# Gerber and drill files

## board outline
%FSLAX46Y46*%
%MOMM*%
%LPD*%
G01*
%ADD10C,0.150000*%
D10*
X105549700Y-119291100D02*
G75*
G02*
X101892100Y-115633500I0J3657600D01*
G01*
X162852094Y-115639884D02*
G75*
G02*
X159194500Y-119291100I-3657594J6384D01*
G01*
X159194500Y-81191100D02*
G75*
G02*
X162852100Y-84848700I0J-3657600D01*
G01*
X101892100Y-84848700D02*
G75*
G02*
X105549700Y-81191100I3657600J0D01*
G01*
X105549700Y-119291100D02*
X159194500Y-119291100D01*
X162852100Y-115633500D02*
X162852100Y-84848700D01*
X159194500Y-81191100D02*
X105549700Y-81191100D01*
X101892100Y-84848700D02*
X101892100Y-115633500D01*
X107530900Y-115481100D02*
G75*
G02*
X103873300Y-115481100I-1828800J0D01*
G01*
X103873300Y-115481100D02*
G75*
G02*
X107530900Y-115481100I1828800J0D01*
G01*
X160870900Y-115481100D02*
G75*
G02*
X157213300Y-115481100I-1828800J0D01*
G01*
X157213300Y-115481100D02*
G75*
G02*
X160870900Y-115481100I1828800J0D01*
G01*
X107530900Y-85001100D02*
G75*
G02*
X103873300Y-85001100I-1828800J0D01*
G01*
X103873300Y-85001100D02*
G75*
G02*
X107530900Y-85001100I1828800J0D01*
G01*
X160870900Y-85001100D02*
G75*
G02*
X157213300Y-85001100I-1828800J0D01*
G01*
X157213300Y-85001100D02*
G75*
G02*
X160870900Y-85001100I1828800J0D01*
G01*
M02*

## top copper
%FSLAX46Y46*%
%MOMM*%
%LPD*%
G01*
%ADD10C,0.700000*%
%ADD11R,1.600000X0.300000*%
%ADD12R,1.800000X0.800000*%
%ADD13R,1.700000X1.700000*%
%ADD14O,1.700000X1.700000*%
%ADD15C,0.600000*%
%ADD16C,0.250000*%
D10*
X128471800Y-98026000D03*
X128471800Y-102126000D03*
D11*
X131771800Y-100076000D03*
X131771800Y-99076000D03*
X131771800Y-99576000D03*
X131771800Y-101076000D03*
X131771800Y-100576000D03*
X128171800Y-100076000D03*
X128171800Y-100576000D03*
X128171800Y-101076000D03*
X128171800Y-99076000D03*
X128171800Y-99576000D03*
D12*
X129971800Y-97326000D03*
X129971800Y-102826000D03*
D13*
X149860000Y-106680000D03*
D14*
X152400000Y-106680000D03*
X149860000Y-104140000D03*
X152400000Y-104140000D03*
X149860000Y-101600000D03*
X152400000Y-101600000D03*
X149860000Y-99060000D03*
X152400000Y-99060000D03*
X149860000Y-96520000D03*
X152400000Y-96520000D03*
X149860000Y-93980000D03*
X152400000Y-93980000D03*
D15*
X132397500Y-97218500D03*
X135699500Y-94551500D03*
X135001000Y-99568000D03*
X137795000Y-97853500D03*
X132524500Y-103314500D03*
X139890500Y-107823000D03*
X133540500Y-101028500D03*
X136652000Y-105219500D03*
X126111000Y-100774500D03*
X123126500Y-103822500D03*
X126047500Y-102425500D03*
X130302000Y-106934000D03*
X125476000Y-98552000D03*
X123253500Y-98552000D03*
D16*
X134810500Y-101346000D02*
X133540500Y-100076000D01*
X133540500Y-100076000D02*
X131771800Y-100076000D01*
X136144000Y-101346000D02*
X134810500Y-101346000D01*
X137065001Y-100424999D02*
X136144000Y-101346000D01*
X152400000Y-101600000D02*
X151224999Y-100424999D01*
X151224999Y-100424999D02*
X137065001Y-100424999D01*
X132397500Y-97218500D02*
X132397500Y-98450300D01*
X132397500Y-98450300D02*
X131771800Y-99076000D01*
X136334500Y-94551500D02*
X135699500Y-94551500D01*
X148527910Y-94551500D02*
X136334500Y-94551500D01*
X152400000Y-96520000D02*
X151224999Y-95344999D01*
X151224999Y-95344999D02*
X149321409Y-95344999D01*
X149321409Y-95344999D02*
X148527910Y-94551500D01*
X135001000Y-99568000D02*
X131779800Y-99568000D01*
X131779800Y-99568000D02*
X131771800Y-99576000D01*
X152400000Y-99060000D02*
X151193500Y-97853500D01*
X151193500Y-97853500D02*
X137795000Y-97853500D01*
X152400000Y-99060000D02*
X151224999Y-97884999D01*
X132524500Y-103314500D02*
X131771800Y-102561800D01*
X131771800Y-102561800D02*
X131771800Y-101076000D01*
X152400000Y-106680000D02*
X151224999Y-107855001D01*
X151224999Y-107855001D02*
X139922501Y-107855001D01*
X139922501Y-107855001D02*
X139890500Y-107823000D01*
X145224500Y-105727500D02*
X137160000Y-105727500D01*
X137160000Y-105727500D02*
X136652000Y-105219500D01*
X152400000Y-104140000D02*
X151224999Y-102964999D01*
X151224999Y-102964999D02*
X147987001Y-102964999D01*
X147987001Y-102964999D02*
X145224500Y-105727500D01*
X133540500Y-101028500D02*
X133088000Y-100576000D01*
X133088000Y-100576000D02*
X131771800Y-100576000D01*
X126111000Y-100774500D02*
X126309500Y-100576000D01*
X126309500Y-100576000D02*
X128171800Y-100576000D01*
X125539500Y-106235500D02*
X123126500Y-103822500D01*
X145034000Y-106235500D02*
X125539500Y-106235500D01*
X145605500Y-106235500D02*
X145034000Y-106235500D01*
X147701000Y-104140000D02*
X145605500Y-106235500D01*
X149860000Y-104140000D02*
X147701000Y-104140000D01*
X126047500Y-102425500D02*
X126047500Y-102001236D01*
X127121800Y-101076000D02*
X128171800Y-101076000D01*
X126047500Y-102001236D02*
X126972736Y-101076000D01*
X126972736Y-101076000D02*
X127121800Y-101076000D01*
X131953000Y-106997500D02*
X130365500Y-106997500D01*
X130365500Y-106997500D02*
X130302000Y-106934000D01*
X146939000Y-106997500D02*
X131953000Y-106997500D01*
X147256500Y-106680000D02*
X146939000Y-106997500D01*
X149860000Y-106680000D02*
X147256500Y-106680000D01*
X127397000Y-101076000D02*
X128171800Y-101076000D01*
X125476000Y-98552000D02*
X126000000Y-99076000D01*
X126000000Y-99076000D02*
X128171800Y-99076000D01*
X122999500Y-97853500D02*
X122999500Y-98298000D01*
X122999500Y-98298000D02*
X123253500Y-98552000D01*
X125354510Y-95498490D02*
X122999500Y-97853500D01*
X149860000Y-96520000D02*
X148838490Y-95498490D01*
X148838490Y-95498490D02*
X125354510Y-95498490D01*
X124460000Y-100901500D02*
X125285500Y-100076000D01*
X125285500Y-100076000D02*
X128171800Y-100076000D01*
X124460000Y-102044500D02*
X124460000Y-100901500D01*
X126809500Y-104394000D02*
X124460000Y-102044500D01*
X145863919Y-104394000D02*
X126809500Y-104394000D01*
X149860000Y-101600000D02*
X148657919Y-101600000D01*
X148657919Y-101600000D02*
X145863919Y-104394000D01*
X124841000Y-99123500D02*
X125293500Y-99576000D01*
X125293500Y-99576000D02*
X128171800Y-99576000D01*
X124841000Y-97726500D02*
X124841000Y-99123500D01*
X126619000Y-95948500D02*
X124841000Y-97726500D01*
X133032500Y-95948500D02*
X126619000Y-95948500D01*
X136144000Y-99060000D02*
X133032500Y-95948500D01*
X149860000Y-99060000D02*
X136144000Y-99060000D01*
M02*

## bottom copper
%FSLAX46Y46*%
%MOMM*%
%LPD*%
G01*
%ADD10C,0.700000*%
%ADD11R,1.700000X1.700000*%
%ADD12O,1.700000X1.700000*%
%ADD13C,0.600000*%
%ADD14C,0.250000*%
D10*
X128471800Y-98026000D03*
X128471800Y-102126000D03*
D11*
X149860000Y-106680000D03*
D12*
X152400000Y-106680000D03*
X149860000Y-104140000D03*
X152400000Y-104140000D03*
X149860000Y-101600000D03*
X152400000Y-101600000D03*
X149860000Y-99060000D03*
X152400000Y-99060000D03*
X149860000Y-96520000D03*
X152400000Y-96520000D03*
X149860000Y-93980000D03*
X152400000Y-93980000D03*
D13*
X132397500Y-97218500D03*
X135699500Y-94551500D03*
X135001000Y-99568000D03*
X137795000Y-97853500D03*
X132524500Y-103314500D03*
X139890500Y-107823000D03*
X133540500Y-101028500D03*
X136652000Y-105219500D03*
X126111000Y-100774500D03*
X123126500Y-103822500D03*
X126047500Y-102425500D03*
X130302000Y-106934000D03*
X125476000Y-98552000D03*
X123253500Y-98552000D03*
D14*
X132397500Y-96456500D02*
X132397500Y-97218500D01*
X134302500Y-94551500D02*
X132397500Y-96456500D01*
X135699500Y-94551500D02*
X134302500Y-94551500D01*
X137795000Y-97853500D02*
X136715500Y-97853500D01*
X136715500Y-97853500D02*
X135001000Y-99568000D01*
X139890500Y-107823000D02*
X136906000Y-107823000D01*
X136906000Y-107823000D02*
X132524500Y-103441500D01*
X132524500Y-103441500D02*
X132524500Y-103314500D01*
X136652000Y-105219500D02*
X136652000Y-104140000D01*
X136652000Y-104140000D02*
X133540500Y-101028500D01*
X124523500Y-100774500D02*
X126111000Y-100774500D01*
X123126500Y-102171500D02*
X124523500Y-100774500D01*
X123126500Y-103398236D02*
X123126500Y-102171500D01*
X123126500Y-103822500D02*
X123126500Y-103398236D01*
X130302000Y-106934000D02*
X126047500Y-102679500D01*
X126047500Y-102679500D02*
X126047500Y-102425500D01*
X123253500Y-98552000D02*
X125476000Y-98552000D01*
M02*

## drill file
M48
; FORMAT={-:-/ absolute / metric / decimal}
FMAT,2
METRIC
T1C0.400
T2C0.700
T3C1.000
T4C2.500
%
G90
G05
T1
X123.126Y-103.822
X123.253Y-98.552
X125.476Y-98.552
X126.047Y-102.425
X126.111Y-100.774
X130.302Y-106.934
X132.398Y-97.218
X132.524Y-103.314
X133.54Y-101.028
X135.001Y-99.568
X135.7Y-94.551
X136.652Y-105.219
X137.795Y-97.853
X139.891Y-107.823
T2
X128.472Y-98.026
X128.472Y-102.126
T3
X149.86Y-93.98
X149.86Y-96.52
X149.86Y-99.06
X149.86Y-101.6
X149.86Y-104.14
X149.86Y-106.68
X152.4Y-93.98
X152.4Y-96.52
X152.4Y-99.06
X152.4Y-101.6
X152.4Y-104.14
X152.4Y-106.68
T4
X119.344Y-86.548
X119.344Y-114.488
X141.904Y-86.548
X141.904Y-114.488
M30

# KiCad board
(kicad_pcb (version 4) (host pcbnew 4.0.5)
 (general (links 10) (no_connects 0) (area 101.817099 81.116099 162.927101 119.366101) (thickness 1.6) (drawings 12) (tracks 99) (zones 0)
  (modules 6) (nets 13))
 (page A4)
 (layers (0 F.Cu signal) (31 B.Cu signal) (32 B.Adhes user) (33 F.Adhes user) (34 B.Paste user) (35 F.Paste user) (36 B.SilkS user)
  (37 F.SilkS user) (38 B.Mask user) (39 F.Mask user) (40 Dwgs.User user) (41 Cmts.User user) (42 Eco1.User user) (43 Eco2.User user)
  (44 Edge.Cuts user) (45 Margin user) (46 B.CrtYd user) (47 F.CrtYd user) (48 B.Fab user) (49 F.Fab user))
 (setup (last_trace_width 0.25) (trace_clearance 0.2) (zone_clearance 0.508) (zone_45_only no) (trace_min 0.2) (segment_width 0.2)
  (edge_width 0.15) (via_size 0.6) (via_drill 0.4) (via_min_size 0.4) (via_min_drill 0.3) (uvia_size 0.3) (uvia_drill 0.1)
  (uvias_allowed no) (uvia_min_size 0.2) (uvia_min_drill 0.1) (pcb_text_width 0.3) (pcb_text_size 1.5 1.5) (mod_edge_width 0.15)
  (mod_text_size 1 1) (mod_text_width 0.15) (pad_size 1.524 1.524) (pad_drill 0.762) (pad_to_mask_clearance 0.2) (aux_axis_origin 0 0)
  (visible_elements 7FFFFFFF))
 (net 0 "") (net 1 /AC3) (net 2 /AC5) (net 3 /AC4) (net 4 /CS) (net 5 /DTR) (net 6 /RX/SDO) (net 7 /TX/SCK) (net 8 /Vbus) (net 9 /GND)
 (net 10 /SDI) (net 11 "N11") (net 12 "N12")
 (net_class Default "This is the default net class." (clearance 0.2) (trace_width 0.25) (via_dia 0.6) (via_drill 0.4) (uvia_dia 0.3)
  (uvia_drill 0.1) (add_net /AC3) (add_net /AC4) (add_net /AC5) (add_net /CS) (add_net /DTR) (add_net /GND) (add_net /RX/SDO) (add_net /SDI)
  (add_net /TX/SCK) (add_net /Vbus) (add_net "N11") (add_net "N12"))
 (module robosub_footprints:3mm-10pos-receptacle (layer F.Cu) (at 129.9718 100.076 90)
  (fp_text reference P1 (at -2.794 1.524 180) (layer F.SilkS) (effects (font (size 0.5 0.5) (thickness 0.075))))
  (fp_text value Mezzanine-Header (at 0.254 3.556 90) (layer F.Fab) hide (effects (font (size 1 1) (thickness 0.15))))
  (pad "" thru_hole circle (at 2.05 -1.5 90) (size 0.7 0.7) (drill 0.7) (layers *.Cu *.Mask))
  (pad "" thru_hole circle (at -2.05 -1.5 90) (size 0.7 0.7) (drill 0.7) (layers *.Cu *.Mask))
  (pad 6 smd rect (at 0 1.8 90) (size 0.3 1.6) (layers F.Cu F.Paste F.Mask) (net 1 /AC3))
  (pad 10 smd rect (at 1 1.8 90) (size 0.3 1.6) (layers F.Cu F.Paste F.Mask) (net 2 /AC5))
  (pad 8 smd rect (at 0.5 1.8 90) (size 0.3 1.6) (layers F.Cu F.Paste F.Mask) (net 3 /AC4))
  (pad 2 smd rect (at -1 1.8 90) (size 0.3 1.6) (layers F.Cu F.Paste F.Mask) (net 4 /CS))
  (pad 4 smd rect (at -0.5 1.8 90) (size 0.3 1.6) (layers F.Cu F.Paste F.Mask) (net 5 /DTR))
  (pad 5 smd rect (at 0 -1.8 90) (size 0.3 1.6) (layers F.Cu F.Paste F.Mask) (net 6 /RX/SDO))
  (pad 3 smd rect (at -0.5 -1.8 90) (size 0.3 1.6) (layers F.Cu F.Paste F.Mask) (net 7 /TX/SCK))
  (pad 1 smd rect (at -1 -1.8 90) (size 0.3 1.6) (layers F.Cu F.Paste F.Mask) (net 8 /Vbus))
  (pad 9 smd rect (at 1 -1.8 90) (size 0.3 1.6) (layers F.Cu F.Paste F.Mask) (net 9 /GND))
  (pad 7 smd rect (at 0.5 -1.8 90) (size 0.3 1.6) (layers F.Cu F.Paste F.Mask) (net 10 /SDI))
  (pad "" smd rect (at 2.75 0 90) (size 0.8 1.8) (layers F.Cu F.Paste F.Mask))
  (pad "" smd rect (at -2.75 0 90) (size 0.8 1.8) (layers F.Cu F.Paste F.Mask)))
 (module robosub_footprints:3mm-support (layer F.Cu) (at 119.3442 86.548204)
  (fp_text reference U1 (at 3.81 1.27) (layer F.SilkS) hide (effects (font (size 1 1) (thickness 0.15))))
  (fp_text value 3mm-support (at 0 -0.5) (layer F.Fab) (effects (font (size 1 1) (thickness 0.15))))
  (pad "" np_thru_hole circle (at 0 0) (size 2.5 2.5) (drill 2.5) (layers *.Cu *.Mask)))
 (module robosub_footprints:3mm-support (layer F.Cu) (at 141.9042 86.548204)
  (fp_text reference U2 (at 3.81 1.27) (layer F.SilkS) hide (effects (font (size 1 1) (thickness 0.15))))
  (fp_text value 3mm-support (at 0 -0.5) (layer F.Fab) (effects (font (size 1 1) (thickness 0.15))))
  (pad "" np_thru_hole circle (at 0 0) (size 2.5 2.5) (drill 2.5) (layers *.Cu *.Mask)))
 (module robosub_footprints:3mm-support (layer F.Cu) (at 119.3442 114.488204)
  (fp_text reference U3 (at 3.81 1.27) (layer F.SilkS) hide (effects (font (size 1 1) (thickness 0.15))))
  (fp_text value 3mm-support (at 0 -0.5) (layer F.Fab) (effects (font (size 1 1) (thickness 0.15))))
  (pad "" np_thru_hole circle (at 0 0) (size 2.5 2.5) (drill 2.5) (layers *.Cu *.Mask)))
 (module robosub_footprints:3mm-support (layer F.Cu) (at 141.9042 114.488204)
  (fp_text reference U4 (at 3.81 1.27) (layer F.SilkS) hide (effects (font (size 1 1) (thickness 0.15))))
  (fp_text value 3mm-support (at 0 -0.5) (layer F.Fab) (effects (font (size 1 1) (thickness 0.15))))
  (pad "" np_thru_hole circle (at 0 0) (size 2.5 2.5) (drill 2.5) (layers *.Cu *.Mask)))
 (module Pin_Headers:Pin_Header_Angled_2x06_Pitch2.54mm (layer B.Cu) (at 149.86 106.68)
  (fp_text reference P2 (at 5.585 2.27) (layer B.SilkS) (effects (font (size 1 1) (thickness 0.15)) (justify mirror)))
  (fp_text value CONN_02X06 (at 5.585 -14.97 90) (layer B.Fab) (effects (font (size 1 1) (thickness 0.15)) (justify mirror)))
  (pad 1 thru_hole rect (at 0 0) (size 1.7 1.7) (drill 1) (layers *.Cu *.Mask) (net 8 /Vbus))
  (pad 2 thru_hole oval (at 2.54 0) (size 1.7 1.7) (drill 1) (layers *.Cu *.Mask) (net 4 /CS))
  (pad 3 thru_hole oval (at 0 -2.54) (size 1.7 1.7) (drill 1) (layers *.Cu *.Mask) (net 7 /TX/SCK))
  (pad 4 thru_hole oval (at 2.54 -2.54) (size 1.7 1.7) (drill 1) (layers *.Cu *.Mask) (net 5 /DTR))
  (pad 5 thru_hole oval (at 0 -5.08) (size 1.7 1.7) (drill 1) (layers *.Cu *.Mask) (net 6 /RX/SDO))
  (pad 6 thru_hole oval (at 2.54 -5.08) (size 1.7 1.7) (drill 1) (layers *.Cu *.Mask) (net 1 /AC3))
  (pad 7 thru_hole oval (at 0 -7.62) (size 1.7 1.7) (drill 1) (layers *.Cu *.Mask) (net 10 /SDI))
  (pad 8 thru_hole oval (at 2.54 -7.62) (size 1.7 1.7) (drill 1) (layers *.Cu *.Mask) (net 3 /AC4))
  (pad 9 thru_hole oval (at 0 -10.16) (size 1.7 1.7) (drill 1) (layers *.Cu *.Mask) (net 9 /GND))
  (pad 10 thru_hole oval (at 2.54 -10.16) (size 1.7 1.7) (drill 1) (layers *.Cu *.Mask) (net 2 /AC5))
  (pad 11 thru_hole oval (at 0 -12.7) (size 1.7 1.7) (drill 1) (layers *.Cu *.Mask) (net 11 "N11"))
  (pad 12 thru_hole oval (at 2.54 -12.7) (size 1.7 1.7) (drill 1) (layers *.Cu *.Mask) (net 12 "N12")))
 (gr_arc (start 105.5497 115.6335) (end 101.8921 115.6335) (angle -90) (layer Edge.Cuts) (width 0.15))
 (gr_arc (start 159.1945 115.6335) (end 159.1945 119.2911) (angle -89.9) (layer Edge.Cuts) (width 0.15))
 (gr_arc (start 159.1945 84.8487) (end 162.8521 84.8487) (angle -90) (layer Edge.Cuts) (width 0.15))
 (gr_arc (start 105.5497 84.8487) (end 105.5497 81.1911) (angle -90) (layer Edge.Cuts) (width 0.15))
 (gr_line (start 105.5497 119.2911) (end 159.1945 119.2911) (layer Edge.Cuts) (width 0.15))
 (gr_line (start 162.8521 115.6335) (end 162.8521 84.8487) (layer Edge.Cuts) (width 0.15))
 (gr_line (start 159.1945 81.1911) (end 105.5497 81.1911) (layer Edge.Cuts) (width 0.15))
 (gr_line (start 101.8921 84.8487) (end 101.8921 115.6335) (layer Edge.Cuts) (width 0.15))
 (gr_circle (center 105.7021 115.4811) (end 107.5309 115.4811) (layer Edge.Cuts) (width 0.15))
 (gr_circle (center 159.0421 115.4811) (end 160.8709 115.4811) (layer Edge.Cuts) (width 0.15))
 (gr_circle (center 105.7021 85.0011) (end 107.5309 85.0011) (layer Edge.Cuts) (width 0.15))
 (gr_circle (center 159.0421 85.0011) (end 160.8709 85.0011) (layer Edge.Cuts) (width 0.15))
 (segment (start 134.8105 101.346) (end 133.5405 100.076) (width 0.25) (layer F.Cu) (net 1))
 (segment (start 133.5405 100.076) (end 131.7718 100.076) (width 0.25) (layer F.Cu) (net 1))
 (segment (start 136.144 101.346) (end 134.8105 101.346) (width 0.25) (layer F.Cu) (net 1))
 (segment (start 137.065001 100.424999) (end 136.144 101.346) (width 0.25) (layer F.Cu) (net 1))
 (segment (start 152.4 101.6) (end 151.224999 100.424999) (width 0.25) (layer F.Cu) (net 1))
 (segment (start 151.224999 100.424999) (end 137.065001 100.424999) (width 0.25) (layer F.Cu) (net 1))
 (segment (start 132.3975 97.2185) (end 132.3975 98.4503) (width 0.25) (layer F.Cu) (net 2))
 (segment (start 132.3975 98.4503) (end 131.7718 99.076) (width 0.25) (layer F.Cu) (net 2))
 (segment (start 132.3975 96.4565) (end 132.3975 97.2185) (width 0.25) (layer B.Cu) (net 2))
 (via (at 132.3975 97.2185) (size 0.6) (drill 0.4) (layers F.Cu B.Cu) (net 2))
 (segment (start 134.3025 94.5515) (end 132.3975 96.4565) (width 0.25) (layer B.Cu) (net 2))
 (segment (start 135.6995 94.5515) (end 134.3025 94.5515) (width 0.25) (layer B.Cu) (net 2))
 (segment (start 136.3345 94.5515) (end 135.6995 94.5515) (width 0.25) (layer F.Cu) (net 2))
 (via (at 135.6995 94.5515) (size 0.6) (drill 0.4) (layers F.Cu B.Cu) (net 2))
 (segment (start 148.52791 94.5515) (end 136.3345 94.5515) (width 0.25) (layer F.Cu) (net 2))
 (segment (start 152.4 96.52) (end 151.224999 95.344999) (width 0.25) (layer F.Cu) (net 2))
 (segment (start 151.224999 95.344999) (end 149.321409 95.344999) (width 0.25) (layer F.Cu) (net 2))
 (segment (start 149.321409 95.344999) (end 148.52791 94.5515) (width 0.25) (layer F.Cu) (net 2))
 (segment (start 135.001 99.568) (end 131.7798 99.568) (width 0.25) (layer F.Cu) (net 3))
 (segment (start 131.7798 99.568) (end 131.7718 99.576) (width 0.25) (layer F.Cu) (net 3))
 (segment (start 137.795 97.8535) (end 136.7155 97.8535) (width 0.25) (layer B.Cu) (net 3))
 (segment (start 136.7155 97.8535) (end 135.001 99.568) (width 0.25) (layer B.Cu) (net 3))
 (via (at 135.001 99.568) (size 0.6) (drill 0.4) (layers F.Cu B.Cu) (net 3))
 (segment (start 152.4 99.06) (end 151.1935 97.8535) (width 0.25) (layer F.Cu) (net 3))
 (segment (start 151.1935 97.8535) (end 137.795 97.8535) (width 0.25) (layer F.Cu) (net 3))
 (via (at 137.795 97.8535) (size 0.6) (drill 0.4) (layers F.Cu B.Cu) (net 3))
 (segment (start 152.4 99.06) (end 151.224999 97.884999) (width 0.25) (layer F.Cu) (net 3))
 (segment (start 132.5245 103.3145) (end 131.7718 102.5618) (width 0.25) (layer F.Cu) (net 4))
 (segment (start 131.7718 102.5618) (end 131.7718 101.076) (width 0.25) (layer F.Cu) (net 4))
 (segment (start 139.8905 107.823) (end 136.906 107.823) (width 0.25) (layer B.Cu) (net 4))
 (segment (start 136.906 107.823) (end 132.5245 103.4415) (width 0.25) (layer B.Cu) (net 4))
 (segment (start 132.5245 103.4415) (end 132.5245 103.3145) (width 0.25) (layer B.Cu) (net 4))
 (via (at 132.5245 103.3145) (size 0.6) (drill 0.4) (layers F.Cu B.Cu) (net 4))
 (segment (start 152.4 106.68) (end 151.224999 107.855001) (width 0.25) (layer F.Cu) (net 4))
 (segment (start 151.224999 107.855001) (end 139.922501 107.855001) (width 0.25) (layer F.Cu) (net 4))
 (segment (start 139.922501 107.855001) (end 139.8905 107.823) (width 0.25) (layer F.Cu) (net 4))
 (via (at 139.8905 107.823) (size 0.6) (drill 0.4) (layers F.Cu B.Cu) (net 4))
 (segment (start 145.2245 105.7275) (end 137.16 105.7275) (width 0.25) (layer F.Cu) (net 5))
 (segment (start 137.16 105.7275) (end 136.652 105.2195) (width 0.25) (layer F.Cu) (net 5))
 (segment (start 152.4 104.14) (end 151.224999 102.964999) (width 0.25) (layer F.Cu) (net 5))
 (segment (start 151.224999 102.964999) (end 147.987001 102.964999) (width 0.25) (layer F.Cu) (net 5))
 (segment (start 147.987001 102.964999) (end 145.2245 105.7275) (width 0.25) (layer F.Cu) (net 5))
 (segment (start 133.5405 101.0285) (end 133.088 100.576) (width 0.25) (layer F.Cu) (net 5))
 (segment (start 133.088 100.576) (end 131.7718 100.576) (width 0.25) (layer F.Cu) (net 5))
 (segment (start 136.652 105.2195) (end 136.652 104.14) (width 0.25) (layer B.Cu) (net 5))
 (segment (start 136.652 104.14) (end 133.5405 101.0285) (width 0.25) (layer B.Cu) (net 5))
 (via (at 133.5405 101.0285) (size 0.6) (drill 0.4) (layers F.Cu B.Cu) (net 5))
 (via (at 136.652 105.2195) (size 0.6) (drill 0.4) (layers F.Cu B.Cu) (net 5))
 (segment (start 126.111 100.7745) (end 126.3095 100.576) (width 0.25) (layer F.Cu) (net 7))
 (segment (start 126.3095 100.576) (end 128.1718 100.576) (width 0.25) (layer F.Cu) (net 7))
 (segment (start 124.5235 100.7745) (end 126.111 100.7745) (width 0.25) (layer B.Cu) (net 7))
 (via (at 126.111 100.7745) (size 0.6) (drill 0.4) (layers F.Cu B.Cu) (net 7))
 (segment (start 123.1265 102.1715) (end 124.5235 100.7745) (width 0.25) (layer B.Cu) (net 7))
 (segment (start 123.1265 103.398236) (end 123.1265 102.1715) (width 0.25) (layer B.Cu) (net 7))
 (segment (start 123.1265 103.8225) (end 123.1265 103.398236) (width 0.25) (layer B.Cu) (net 7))
 (via (at 123.1265 103.8225) (size 0.6) (drill 0.4) (layers F.Cu B.Cu) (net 7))
 (segment (start 125.5395 106.2355) (end 123.1265 103.8225) (width 0.25) (layer F.Cu) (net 7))
 (segment (start 145.034 106.2355) (end 125.5395 106.2355) (width 0.25) (layer F.Cu) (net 7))
 (segment (start 145.6055 106.2355) (end 145.034 106.2355) (width 0.25) (layer F.Cu) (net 7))
 (segment (start 147.701 104.14) (end 145.6055 106.2355) (width 0.25) (layer F.Cu) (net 7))
 (segment (start 149.86 104.14) (end 147.701 104.14) (width 0.25) (layer F.Cu) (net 7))
 (segment (start 126.0475 102.4255) (end 126.0475 102.001236) (width 0.25) (layer F.Cu) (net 8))
 (segment (start 127.1218 101.076) (end 128.1718 101.076) (width 0.25) (layer F.Cu) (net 8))
 (segment (start 126.0475 102.001236) (end 126.972736 101.076) (width 0.25) (layer F.Cu) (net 8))
 (segment (start 126.972736 101.076) (end 127.1218 101.076) (width 0.25) (layer F.Cu) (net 8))
 (segment (start 130.302 106.934) (end 126.0475 102.6795) (width 0.25) (layer B.Cu) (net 8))
 (segment (start 126.0475 102.6795) (end 126.0475 102.4255) (width 0.25) (layer B.Cu) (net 8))
 (via (at 126.0475 102.4255) (size 0.6) (drill 0.4) (layers F.Cu B.Cu) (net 8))
 (segment (start 131.953 106.9975) (end 130.3655 106.9975) (width 0.25) (layer F.Cu) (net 8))
 (segment (start 130.3655 106.9975) (end 130.302 106.934) (width 0.25) (layer F.Cu) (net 8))
 (via (at 130.302 106.934) (size 0.6) (drill 0.4) (layers F.Cu B.Cu) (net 8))
 (segment (start 146.939 106.9975) (end 131.953 106.9975) (width 0.25) (layer F.Cu) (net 8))
 (segment (start 147.2565 106.68) (end 146.939 106.9975) (width 0.25) (layer F.Cu) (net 8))
 (segment (start 149.86 106.68) (end 147.2565 106.68) (width 0.25) (layer F.Cu) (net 8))
 (segment (start 127.397 101.076) (end 128.1718 101.076) (width 0.25) (layer F.Cu) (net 8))
 (segment (start 125.476 98.552) (end 126 99.076) (width 0.25) (layer F.Cu) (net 9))
 (segment (start 126 99.076) (end 128.1718 99.076) (width 0.25) (layer F.Cu) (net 9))
 (segment (start 123.2535 98.552) (end 125.476 98.552) (width 0.25) (layer B.Cu) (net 9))
 (via (at 125.476 98.552) (size 0.6) (drill 0.4) (layers F.Cu B.Cu) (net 9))
 (segment (start 122.9995 97.8535) (end 122.9995 98.298) (width 0.25) (layer F.Cu) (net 9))
 (segment (start 122.9995 98.298) (end 123.2535 98.552) (width 0.25) (layer F.Cu) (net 9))
 (via (at 123.2535 98.552) (size 0.6) (drill 0.4) (layers F.Cu B.Cu) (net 9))
 (segment (start 125.35451 95.49849) (end 122.9995 97.8535) (width 0.25) (layer F.Cu) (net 9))
 (segment (start 149.86 96.52) (end 148.83849 95.49849) (width 0.25) (layer F.Cu) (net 9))
 (segment (start 148.83849 95.49849) (end 125.35451 95.49849) (width 0.25) (layer F.Cu) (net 9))
 (segment (start 124.46 100.9015) (end 125.2855 100.076) (width 0.25) (layer F.Cu) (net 6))
 (segment (start 125.2855 100.076) (end 128.1718 100.076) (width 0.25) (layer F.Cu) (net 6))
 (segment (start 124.46 102.0445) (end 124.46 100.9015) (width 0.25) (layer F.Cu) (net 6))
 (segment (start 126.8095 104.394) (end 124.46 102.0445) (width 0.25) (layer F.Cu) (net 6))
 (segment (start 145.863919 104.394) (end 126.8095 104.394) (width 0.25) (layer F.Cu) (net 6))
 (segment (start 149.86 101.6) (end 148.657919 101.6) (width 0.25) (layer F.Cu) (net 6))
 (segment (start 148.657919 101.6) (end 145.863919 104.394) (width 0.25) (layer F.Cu) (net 6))
 (segment (start 124.841 99.1235) (end 125.2935 99.576) (width 0.25) (layer F.Cu) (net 10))
 (segment (start 125.2935 99.576) (end 128.1718 99.576) (width 0.25) (layer F.Cu) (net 10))
 (segment (start 124.841 97.7265) (end 124.841 99.1235) (width 0.25) (layer F.Cu) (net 10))
 (segment (start 126.619 95.9485) (end 124.841 97.7265) (width 0.25) (layer F.Cu) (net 10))
 (segment (start 133.0325 95.9485) (end 126.619 95.9485) (width 0.25) (layer F.Cu) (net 10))
 (segment (start 136.144 99.06) (end 133.0325 95.9485) (width 0.25) (layer F.Cu) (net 10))
 (segment (start 149.86 99.06) (end 136.144 99.06) (width 0.25) (layer F.Cu) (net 10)))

